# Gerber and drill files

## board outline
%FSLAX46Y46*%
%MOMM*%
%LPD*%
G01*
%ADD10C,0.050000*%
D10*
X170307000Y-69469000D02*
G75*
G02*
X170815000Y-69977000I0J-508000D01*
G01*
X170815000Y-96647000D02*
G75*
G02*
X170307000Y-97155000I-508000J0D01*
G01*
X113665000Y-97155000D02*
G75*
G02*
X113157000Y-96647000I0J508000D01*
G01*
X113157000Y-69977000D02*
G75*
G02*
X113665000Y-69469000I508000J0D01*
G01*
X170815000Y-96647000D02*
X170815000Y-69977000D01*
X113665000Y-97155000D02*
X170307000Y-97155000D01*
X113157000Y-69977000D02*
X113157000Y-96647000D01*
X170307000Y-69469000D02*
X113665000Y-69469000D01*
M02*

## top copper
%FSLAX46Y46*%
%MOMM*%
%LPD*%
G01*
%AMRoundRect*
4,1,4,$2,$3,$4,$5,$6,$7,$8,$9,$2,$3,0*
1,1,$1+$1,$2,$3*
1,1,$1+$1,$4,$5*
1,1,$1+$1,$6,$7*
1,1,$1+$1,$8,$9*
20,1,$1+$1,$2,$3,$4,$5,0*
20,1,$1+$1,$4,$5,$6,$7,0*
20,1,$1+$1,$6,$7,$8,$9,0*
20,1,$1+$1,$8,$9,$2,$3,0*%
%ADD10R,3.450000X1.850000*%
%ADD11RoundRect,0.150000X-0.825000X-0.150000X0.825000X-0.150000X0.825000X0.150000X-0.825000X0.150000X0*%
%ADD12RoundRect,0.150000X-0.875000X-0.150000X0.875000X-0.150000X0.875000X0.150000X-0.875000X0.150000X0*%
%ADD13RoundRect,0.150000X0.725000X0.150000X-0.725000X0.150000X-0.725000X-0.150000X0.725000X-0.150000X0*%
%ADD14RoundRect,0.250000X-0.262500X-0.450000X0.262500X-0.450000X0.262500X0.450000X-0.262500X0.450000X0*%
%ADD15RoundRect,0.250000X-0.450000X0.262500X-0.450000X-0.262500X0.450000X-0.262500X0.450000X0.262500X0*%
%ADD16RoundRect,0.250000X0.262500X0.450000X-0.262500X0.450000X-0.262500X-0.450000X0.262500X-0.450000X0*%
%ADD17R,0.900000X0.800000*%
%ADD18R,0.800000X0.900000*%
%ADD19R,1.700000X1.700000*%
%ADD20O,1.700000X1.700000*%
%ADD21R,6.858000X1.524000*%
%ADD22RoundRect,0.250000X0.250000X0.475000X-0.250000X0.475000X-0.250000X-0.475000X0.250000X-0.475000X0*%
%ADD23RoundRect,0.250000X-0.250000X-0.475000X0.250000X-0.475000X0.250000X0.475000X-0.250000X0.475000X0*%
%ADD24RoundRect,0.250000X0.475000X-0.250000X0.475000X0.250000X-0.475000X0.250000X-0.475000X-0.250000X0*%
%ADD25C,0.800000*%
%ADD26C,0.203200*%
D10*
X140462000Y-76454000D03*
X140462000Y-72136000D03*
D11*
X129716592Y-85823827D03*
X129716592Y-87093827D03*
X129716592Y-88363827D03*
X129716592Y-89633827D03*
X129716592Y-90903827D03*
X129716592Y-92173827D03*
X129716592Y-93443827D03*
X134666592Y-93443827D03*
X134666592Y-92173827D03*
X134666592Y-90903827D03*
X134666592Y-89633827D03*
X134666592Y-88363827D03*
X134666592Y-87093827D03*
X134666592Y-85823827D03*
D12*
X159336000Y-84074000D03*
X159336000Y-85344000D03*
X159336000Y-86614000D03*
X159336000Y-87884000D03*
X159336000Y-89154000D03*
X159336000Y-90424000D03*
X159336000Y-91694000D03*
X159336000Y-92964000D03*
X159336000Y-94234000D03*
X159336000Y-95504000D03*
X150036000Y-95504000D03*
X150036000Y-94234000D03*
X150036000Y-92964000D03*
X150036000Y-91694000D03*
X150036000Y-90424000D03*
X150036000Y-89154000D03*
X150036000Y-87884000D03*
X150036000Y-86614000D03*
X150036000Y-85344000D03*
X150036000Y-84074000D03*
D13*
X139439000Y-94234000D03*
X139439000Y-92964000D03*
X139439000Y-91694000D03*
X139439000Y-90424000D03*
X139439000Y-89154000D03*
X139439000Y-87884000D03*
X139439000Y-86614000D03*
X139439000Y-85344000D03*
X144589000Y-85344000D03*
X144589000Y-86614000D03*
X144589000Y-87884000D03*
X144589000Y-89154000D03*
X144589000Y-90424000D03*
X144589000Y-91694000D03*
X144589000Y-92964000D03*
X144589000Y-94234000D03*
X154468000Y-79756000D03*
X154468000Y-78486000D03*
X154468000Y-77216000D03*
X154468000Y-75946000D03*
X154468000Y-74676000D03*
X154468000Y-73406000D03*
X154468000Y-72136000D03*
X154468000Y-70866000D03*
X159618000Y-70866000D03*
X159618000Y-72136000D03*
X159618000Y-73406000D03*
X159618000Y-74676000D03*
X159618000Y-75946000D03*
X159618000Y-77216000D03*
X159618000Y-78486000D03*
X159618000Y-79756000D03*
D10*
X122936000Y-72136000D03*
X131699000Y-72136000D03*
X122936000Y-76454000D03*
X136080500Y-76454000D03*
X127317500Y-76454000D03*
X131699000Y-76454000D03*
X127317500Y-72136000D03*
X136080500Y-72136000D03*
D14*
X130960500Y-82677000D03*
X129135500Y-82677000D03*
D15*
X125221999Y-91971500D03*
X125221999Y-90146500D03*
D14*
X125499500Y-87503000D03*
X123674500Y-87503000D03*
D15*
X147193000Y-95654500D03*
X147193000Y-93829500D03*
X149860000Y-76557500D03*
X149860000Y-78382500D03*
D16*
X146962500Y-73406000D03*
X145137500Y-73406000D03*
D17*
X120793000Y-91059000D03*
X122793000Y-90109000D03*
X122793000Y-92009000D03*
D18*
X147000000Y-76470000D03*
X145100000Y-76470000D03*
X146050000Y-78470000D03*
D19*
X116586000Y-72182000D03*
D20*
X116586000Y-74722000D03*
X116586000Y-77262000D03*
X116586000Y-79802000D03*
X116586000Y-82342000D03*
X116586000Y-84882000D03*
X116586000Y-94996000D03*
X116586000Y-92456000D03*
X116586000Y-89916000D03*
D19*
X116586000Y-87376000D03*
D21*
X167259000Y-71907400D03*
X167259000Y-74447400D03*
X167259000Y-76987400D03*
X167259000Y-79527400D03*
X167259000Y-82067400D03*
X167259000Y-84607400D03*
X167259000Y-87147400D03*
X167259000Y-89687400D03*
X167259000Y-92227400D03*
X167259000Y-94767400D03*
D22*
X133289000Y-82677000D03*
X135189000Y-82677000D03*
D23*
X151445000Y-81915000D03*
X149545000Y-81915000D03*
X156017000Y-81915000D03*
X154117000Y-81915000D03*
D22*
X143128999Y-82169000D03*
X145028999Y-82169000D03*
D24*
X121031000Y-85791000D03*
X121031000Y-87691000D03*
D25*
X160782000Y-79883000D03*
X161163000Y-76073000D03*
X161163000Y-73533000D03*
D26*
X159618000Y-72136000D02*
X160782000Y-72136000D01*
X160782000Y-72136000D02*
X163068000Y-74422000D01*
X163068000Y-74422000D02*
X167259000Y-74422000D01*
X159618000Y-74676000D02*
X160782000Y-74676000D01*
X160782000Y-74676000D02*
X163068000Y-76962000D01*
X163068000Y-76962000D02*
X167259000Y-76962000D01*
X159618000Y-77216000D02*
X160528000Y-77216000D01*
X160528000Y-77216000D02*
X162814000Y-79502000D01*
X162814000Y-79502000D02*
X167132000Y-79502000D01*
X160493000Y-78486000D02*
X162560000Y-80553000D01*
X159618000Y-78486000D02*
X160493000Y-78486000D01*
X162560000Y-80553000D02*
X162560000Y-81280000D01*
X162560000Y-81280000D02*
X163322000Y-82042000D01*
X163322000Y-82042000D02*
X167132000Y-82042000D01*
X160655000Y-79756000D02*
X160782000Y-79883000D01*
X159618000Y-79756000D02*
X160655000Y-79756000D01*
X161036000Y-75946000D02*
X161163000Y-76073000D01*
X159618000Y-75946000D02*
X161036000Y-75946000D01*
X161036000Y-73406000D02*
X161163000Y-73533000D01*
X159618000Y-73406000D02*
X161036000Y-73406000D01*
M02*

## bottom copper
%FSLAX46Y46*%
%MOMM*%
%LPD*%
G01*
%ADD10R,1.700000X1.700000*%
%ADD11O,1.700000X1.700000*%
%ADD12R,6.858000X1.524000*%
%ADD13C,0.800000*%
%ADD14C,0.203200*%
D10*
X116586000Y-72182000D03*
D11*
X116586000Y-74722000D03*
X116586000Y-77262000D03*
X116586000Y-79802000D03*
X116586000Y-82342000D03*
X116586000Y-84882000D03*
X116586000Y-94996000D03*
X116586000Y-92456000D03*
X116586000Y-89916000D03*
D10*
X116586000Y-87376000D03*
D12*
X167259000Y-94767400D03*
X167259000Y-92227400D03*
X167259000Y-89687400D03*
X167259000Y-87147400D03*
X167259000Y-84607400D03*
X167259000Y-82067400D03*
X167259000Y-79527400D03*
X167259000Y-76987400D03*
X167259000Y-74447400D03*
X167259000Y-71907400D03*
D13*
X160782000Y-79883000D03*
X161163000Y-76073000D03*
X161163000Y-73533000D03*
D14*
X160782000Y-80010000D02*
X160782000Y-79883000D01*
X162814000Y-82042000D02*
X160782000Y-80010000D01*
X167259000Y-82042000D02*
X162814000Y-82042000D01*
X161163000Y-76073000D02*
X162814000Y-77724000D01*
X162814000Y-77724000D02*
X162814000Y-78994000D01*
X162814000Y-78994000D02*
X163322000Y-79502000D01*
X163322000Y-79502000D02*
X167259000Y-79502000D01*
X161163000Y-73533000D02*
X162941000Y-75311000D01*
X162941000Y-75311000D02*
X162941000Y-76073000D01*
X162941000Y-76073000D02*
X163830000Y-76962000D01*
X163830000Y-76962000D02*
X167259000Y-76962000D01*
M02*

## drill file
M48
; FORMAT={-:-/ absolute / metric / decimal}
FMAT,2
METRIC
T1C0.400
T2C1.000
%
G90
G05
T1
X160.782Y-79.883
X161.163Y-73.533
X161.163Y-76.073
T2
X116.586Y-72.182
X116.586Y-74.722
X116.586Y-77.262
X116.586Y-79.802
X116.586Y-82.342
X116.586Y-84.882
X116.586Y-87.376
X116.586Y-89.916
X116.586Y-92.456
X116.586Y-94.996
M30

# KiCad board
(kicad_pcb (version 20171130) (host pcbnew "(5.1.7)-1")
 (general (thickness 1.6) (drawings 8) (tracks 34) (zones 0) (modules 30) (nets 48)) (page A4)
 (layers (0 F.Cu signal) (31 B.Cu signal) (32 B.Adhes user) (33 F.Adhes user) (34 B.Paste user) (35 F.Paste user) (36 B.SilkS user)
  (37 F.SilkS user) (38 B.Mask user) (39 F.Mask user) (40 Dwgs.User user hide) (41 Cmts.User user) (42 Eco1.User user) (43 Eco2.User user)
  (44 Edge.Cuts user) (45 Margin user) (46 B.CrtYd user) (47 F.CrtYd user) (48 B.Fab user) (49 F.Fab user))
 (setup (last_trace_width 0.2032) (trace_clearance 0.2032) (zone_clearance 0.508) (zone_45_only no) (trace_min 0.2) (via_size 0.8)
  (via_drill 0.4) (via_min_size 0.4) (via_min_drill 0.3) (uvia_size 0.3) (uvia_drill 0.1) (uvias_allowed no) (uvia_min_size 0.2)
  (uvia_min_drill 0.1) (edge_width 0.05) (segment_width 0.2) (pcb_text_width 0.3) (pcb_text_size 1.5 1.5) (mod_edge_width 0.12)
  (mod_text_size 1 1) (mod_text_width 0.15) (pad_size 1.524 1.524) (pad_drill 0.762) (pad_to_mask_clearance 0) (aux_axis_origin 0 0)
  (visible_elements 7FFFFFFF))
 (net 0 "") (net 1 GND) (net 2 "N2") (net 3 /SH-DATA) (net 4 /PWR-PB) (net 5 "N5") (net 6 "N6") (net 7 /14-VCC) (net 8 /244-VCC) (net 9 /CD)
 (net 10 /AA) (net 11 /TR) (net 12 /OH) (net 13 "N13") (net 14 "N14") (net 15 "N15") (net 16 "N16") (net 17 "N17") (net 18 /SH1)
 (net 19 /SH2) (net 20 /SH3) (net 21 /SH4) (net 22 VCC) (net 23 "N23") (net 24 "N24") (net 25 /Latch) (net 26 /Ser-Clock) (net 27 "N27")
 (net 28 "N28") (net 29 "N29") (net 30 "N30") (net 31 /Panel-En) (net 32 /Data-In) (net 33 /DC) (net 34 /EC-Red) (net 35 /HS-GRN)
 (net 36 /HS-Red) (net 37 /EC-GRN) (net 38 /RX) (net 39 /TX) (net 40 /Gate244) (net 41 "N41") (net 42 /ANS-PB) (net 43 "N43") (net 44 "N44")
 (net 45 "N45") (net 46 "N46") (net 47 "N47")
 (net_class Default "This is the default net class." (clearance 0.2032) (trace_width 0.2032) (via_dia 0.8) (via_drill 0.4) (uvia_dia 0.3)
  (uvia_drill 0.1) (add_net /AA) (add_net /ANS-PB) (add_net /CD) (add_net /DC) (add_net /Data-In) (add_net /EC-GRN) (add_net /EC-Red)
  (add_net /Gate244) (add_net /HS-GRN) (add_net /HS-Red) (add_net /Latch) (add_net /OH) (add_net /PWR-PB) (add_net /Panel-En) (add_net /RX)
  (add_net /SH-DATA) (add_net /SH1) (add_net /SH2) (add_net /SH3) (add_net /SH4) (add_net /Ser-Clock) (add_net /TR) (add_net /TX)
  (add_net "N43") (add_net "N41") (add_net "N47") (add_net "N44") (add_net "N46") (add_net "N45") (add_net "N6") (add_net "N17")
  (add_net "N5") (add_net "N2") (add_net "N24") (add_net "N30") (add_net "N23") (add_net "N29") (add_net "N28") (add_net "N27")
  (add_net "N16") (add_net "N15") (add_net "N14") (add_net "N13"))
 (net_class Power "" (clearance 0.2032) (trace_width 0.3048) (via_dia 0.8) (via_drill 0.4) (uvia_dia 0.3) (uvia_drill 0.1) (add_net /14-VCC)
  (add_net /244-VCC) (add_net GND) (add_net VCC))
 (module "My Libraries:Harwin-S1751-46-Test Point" (layer F.Cu) (at 140.462 76.454)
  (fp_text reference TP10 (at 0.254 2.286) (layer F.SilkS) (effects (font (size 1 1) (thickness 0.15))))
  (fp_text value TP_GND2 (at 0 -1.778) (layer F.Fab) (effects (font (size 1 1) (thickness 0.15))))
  (pad 1 smd rect (at 0 0) (size 3.45 1.85) (layers F.Cu F.Paste F.Mask) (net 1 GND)))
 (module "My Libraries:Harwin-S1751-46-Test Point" (layer F.Cu) (at 140.462 72.136)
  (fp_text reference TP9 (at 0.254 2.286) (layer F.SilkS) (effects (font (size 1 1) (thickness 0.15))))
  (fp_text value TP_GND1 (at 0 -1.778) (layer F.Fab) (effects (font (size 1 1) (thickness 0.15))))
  (pad 1 smd rect (at 0 0) (size 3.45 1.85) (layers F.Cu F.Paste F.Mask) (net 1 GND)))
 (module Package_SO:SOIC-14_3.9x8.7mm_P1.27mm (layer F.Cu) (at 132.191592 89.633827)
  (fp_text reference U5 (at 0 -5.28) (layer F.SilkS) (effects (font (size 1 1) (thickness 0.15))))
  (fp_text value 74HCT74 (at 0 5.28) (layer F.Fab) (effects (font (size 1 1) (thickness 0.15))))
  (pad 1 smd roundrect (at -2.475 -3.81) (size 1.95 0.6) (layers F.Cu F.Paste F.Mask) (roundrect_rratio 0.25) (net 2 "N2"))
  (pad 2 smd roundrect (at -2.475 -2.54) (size 1.95 0.6) (layers F.Cu F.Paste F.Mask) (roundrect_rratio 0.25) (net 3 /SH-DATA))
  (pad 3 smd roundrect (at -2.475 -1.27) (size 1.95 0.6) (layers F.Cu F.Paste F.Mask) (roundrect_rratio 0.25) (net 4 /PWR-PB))
  (pad 4 smd roundrect (at -2.475 0) (size 1.95 0.6) (layers F.Cu F.Paste F.Mask) (roundrect_rratio 0.25) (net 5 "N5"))
  (pad 5 smd roundrect (at -2.475 1.27) (size 1.95 0.6) (layers F.Cu F.Paste F.Mask) (roundrect_rratio 0.25) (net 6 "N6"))
  (pad 6 smd roundrect (at -2.475 2.54) (size 1.95 0.6) (layers F.Cu F.Paste F.Mask) (roundrect_rratio 0.25) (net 3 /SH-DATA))
  (pad 7 smd roundrect (at -2.475 3.81) (size 1.95 0.6) (layers F.Cu F.Paste F.Mask) (roundrect_rratio 0.25) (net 1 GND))
  (pad 8 smd roundrect (at 2.475 3.81) (size 1.95 0.6) (layers F.Cu F.Paste F.Mask) (roundrect_rratio 0.25))
  (pad 9 smd roundrect (at 2.475 2.54) (size 1.95 0.6) (layers F.Cu F.Paste F.Mask) (roundrect_rratio 0.25))
  (pad 10 smd roundrect (at 2.475 1.27) (size 1.95 0.6) (layers F.Cu F.Paste F.Mask) (roundrect_rratio 0.25))
  (pad 11 smd roundrect (at 2.475 0) (size 1.95 0.6) (layers F.Cu F.Paste F.Mask) (roundrect_rratio 0.25))
  (pad 12 smd roundrect (at 2.475 -1.27) (size 1.95 0.6) (layers F.Cu F.Paste F.Mask) (roundrect_rratio 0.25))
  (pad 13 smd roundrect (at 2.475 -2.54) (size 1.95 0.6) (layers F.Cu F.Paste F.Mask) (roundrect_rratio 0.25))
  (pad 14 smd roundrect (at 2.475 -3.81) (size 1.95 0.6) (layers F.Cu F.Paste F.Mask) (roundrect_rratio 0.25) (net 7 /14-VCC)))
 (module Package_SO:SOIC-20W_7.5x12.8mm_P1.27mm (layer F.Cu) (at 154.686 89.789)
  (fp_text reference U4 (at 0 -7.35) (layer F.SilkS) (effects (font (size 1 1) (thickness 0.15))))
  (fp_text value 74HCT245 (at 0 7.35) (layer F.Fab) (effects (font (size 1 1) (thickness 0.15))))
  (pad 20 smd roundrect (at 4.65 -5.715) (size 2.05 0.6) (layers F.Cu F.Paste F.Mask) (roundrect_rratio 0.25) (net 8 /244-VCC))
  (pad 19 smd roundrect (at 4.65 -4.445) (size 2.05 0.6) (layers F.Cu F.Paste F.Mask) (roundrect_rratio 0.25) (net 1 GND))
  (pad 18 smd roundrect (at 4.65 -3.175) (size 2.05 0.6) (layers F.Cu F.Paste F.Mask) (roundrect_rratio 0.25) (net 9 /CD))
  (pad 17 smd roundrect (at 4.65 -1.905) (size 2.05 0.6) (layers F.Cu F.Paste F.Mask) (roundrect_rratio 0.25) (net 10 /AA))
  (pad 16 smd roundrect (at 4.65 -0.635) (size 2.05 0.6) (layers F.Cu F.Paste F.Mask) (roundrect_rratio 0.25) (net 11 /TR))
  (pad 15 smd roundrect (at 4.65 0.635) (size 2.05 0.6) (layers F.Cu F.Paste F.Mask) (roundrect_rratio 0.25) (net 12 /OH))
  (pad 14 smd roundrect (at 4.65 1.905) (size 2.05 0.6) (layers F.Cu F.Paste F.Mask) (roundrect_rratio 0.25) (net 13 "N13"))
  (pad 13 smd roundrect (at 4.65 3.175) (size 2.05 0.6) (layers F.Cu F.Paste F.Mask) (roundrect_rratio 0.25) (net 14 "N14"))
  (pad 12 smd roundrect (at 4.65 4.445) (size 2.05 0.6) (layers F.Cu F.Paste F.Mask) (roundrect_rratio 0.25) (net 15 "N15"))
  (pad 11 smd roundrect (at 4.65 5.715) (size 2.05 0.6) (layers F.Cu F.Paste F.Mask) (roundrect_rratio 0.25) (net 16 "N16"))
  (pad 10 smd roundrect (at -4.65 5.715) (size 2.05 0.6) (layers F.Cu F.Paste F.Mask) (roundrect_rratio 0.25) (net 1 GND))
  (pad 9 smd roundrect (at -4.65 4.445) (size 2.05 0.6) (layers F.Cu F.Paste F.Mask) (roundrect_rratio 0.25) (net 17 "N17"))
  (pad 8 smd roundrect (at -4.65 3.175) (size 2.05 0.6) (layers F.Cu F.Paste F.Mask) (roundrect_rratio 0.25) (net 17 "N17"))
  (pad 7 smd roundrect (at -4.65 1.905) (size 2.05 0.6) (layers F.Cu F.Paste F.Mask) (roundrect_rratio 0.25) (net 17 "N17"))
  (pad 6 smd roundrect (at -4.65 0.635) (size 2.05 0.6) (layers F.Cu F.Paste F.Mask) (roundrect_rratio 0.25) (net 17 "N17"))
  (pad 5 smd roundrect (at -4.65 -0.635) (size 2.05 0.6) (layers F.Cu F.Paste F.Mask) (roundrect_rratio 0.25) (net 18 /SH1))
  (pad 4 smd roundrect (at -4.65 -1.905) (size 2.05 0.6) (layers F.Cu F.Paste F.Mask) (roundrect_rratio 0.25) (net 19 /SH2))
  (pad 3 smd roundrect (at -4.65 -3.175) (size 2.05 0.6) (layers F.Cu F.Paste F.Mask) (roundrect_rratio 0.25) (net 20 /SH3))
  (pad 2 smd roundrect (at -4.65 -4.445) (size 2.05 0.6) (layers F.Cu F.Paste F.Mask) (roundrect_rratio 0.25) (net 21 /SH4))
  (pad 1 smd roundrect (at -4.65 -5.715) (size 2.05 0.6) (layers F.Cu F.Paste F.Mask) (roundrect_rratio 0.25) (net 8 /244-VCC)))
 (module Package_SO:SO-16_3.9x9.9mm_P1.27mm (layer F.Cu) (at 142.014 89.789 180)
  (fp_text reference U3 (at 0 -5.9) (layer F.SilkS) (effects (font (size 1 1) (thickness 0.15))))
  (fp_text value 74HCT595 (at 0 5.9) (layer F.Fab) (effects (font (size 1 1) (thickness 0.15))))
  (pad 16 smd roundrect (at 2.575 -4.445 180) (size 1.75 0.6) (layers F.Cu F.Paste F.Mask) (roundrect_rratio 0.25) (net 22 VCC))
  (pad 15 smd roundrect (at 2.575 -3.175 180) (size 1.75 0.6) (layers F.Cu F.Paste F.Mask) (roundrect_rratio 0.25) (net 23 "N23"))
  (pad 14 smd roundrect (at 2.575 -1.905 180) (size 1.75 0.6) (layers F.Cu F.Paste F.Mask) (roundrect_rratio 0.25) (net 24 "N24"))
  (pad 13 smd roundrect (at 2.575 -0.635 180) (size 1.75 0.6) (layers F.Cu F.Paste F.Mask) (roundrect_rratio 0.25) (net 1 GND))
  (pad 12 smd roundrect (at 2.575 0.635 180) (size 1.75 0.6) (layers F.Cu F.Paste F.Mask) (roundrect_rratio 0.25) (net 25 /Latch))
  (pad 11 smd roundrect (at 2.575 1.905 180) (size 1.75 0.6) (layers F.Cu F.Paste F.Mask) (roundrect_rratio 0.25) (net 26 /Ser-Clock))
  (pad 10 smd roundrect (at 2.575 3.175 180) (size 1.75 0.6) (layers F.Cu F.Paste F.Mask) (roundrect_rratio 0.25) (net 22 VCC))
  (pad 9 smd roundrect (at 2.575 4.445 180) (size 1.75 0.6) (layers F.Cu F.Paste F.Mask) (roundrect_rratio 0.25) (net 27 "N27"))
  (pad 8 smd roundrect (at -2.575 4.445 180) (size 1.75 0.6) (layers F.Cu F.Paste F.Mask) (roundrect_rratio 0.25) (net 1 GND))
  (pad 7 smd roundrect (at -2.575 3.175 180) (size 1.75 0.6) (layers F.Cu F.Paste F.Mask) (roundrect_rratio 0.25) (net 21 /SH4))
  (pad 6 smd roundrect (at -2.575 1.905 180) (size 1.75 0.6) (layers F.Cu F.Paste F.Mask) (roundrect_rratio 0.25) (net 20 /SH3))
  (pad 5 smd roundrect (at -2.575 0.635 180) (size 1.75 0.6) (layers F.Cu F.Paste F.Mask) (roundrect_rratio 0.25) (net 19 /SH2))
  (pad 4 smd roundrect (at -2.575 -0.635 180) (size 1.75 0.6) (layers F.Cu F.Paste F.Mask) (roundrect_rratio 0.25) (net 18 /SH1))
  (pad 3 smd roundrect (at -2.575 -1.905 180) (size 1.75 0.6) (layers F.Cu F.Paste F.Mask) (roundrect_rratio 0.25) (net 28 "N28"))
  (pad 2 smd roundrect (at -2.575 -3.175 180) (size 1.75 0.6) (layers F.Cu F.Paste F.Mask) (roundrect_rratio 0.25) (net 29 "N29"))
  (pad 1 smd roundrect (at -2.575 -4.445 180) (size 1.75 0.6) (layers F.Cu F.Paste F.Mask) (roundrect_rratio 0.25) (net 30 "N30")))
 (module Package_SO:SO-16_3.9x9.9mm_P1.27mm (layer F.Cu) (at 157.043 75.311 180)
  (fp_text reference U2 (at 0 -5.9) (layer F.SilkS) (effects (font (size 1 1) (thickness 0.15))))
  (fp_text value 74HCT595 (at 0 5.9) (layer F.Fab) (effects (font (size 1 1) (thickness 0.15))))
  (pad 16 smd roundrect (at 2.575 -4.445 180) (size 1.75 0.6) (layers F.Cu F.Paste F.Mask) (roundrect_rratio 0.25) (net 22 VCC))
  (pad 15 smd roundrect (at 2.575 -3.175 180) (size 1.75 0.6) (layers F.Cu F.Paste F.Mask) (roundrect_rratio 0.25) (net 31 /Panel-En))
  (pad 14 smd roundrect (at 2.575 -1.905 180) (size 1.75 0.6) (layers F.Cu F.Paste F.Mask) (roundrect_rratio 0.25) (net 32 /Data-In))
  (pad 13 smd roundrect (at 2.575 -0.635 180) (size 1.75 0.6) (layers F.Cu F.Paste F.Mask) (roundrect_rratio 0.25) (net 1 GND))
  (pad 12 smd roundrect (at 2.575 0.635 180) (size 1.75 0.6) (layers F.Cu F.Paste F.Mask) (roundrect_rratio 0.25) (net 25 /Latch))
  (pad 11 smd roundrect (at 2.575 1.905 180) (size 1.75 0.6) (layers F.Cu F.Paste F.Mask) (roundrect_rratio 0.25) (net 26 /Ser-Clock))
  (pad 10 smd roundrect (at 2.575 3.175 180) (size 1.75 0.6) (layers F.Cu F.Paste F.Mask) (roundrect_rratio 0.25) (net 22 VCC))
  (pad 9 smd roundrect (at 2.575 4.445 180) (size 1.75 0.6) (layers F.Cu F.Paste F.Mask) (roundrect_rratio 0.25) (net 24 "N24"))
  (pad 8 smd roundrect (at -2.575 4.445 180) (size 1.75 0.6) (layers F.Cu F.Paste F.Mask) (roundrect_rratio 0.25) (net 1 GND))
  (pad 7 smd roundrect (at -2.575 3.175 180) (size 1.75 0.6) (layers F.Cu F.Paste F.Mask) (roundrect_rratio 0.25) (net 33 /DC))
  (pad 6 smd roundrect (at -2.575 1.905 180) (size 1.75 0.6) (layers F.Cu F.Paste F.Mask) (roundrect_rratio 0.25) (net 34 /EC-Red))
  (pad 5 smd roundrect (at -2.575 0.635 180) (size 1.75 0.6) (layers F.Cu F.Paste F.Mask) (roundrect_rratio 0.25) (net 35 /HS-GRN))
  (pad 4 smd roundrect (at -2.575 -0.635 180) (size 1.75 0.6) (layers F.Cu F.Paste F.Mask) (roundrect_rratio 0.25) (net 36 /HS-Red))
  (pad 3 smd roundrect (at -2.575 -1.905 180) (size 1.75 0.6) (layers F.Cu F.Paste F.Mask) (roundrect_rratio 0.25) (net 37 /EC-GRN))
  (pad 2 smd roundrect (at -2.575 -3.175 180) (size 1.75 0.6) (layers F.Cu F.Paste F.Mask) (roundrect_rratio 0.25) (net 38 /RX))
  (pad 1 smd roundrect (at -2.575 -4.445 180) (size 1.75 0.6) (layers F.Cu F.Paste F.Mask) (roundrect_rratio 0.25) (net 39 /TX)))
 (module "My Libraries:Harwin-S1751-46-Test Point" (layer F.Cu) (at 122.936 72.136)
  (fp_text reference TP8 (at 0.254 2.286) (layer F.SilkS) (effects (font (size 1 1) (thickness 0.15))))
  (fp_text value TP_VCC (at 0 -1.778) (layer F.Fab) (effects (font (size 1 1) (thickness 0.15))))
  (pad 1 smd rect (at 0 0) (size 3.45 1.85) (layers F.Cu F.Paste F.Mask) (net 22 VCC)))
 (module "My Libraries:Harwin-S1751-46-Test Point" (layer F.Cu) (at 131.699 72.136)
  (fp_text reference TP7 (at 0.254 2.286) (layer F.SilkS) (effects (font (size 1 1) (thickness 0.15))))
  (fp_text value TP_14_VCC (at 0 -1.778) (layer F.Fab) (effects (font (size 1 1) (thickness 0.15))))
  (pad 1 smd rect (at 0 0) (size 3.45 1.85) (layers F.Cu F.Paste F.Mask) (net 7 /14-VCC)))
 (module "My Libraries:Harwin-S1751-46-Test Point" (layer F.Cu) (at 122.936 76.454)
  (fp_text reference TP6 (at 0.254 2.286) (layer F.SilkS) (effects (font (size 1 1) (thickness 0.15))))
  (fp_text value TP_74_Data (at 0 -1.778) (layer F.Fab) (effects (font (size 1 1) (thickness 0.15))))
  (pad 1 smd rect (at 0 0) (size 3.45 1.85) (layers F.Cu F.Paste F.Mask) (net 3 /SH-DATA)))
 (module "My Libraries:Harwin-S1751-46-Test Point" (layer F.Cu) (at 136.0805 76.454)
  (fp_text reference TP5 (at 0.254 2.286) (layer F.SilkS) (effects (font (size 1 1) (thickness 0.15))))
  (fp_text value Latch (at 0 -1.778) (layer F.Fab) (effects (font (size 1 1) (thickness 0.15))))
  (pad 1 smd rect (at 0 0) (size 3.45 1.85) (layers F.Cu F.Paste F.Mask) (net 25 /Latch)))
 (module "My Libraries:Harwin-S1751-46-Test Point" (layer F.Cu) (at 127.3175 76.454)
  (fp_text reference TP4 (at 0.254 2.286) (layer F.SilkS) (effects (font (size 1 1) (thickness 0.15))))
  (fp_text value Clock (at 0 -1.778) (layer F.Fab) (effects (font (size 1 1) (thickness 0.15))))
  (pad 1 smd rect (at 0 0) (size 3.45 1.85) (layers F.Cu F.Paste F.Mask) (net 26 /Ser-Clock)))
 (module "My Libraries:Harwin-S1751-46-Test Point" (layer F.Cu) (at 131.699 76.454)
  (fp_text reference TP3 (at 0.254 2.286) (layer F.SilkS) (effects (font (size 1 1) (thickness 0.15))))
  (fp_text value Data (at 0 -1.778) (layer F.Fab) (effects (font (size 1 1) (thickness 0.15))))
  (pad 1 smd rect (at 0 0) (size 3.45 1.85) (layers F.Cu F.Paste F.Mask) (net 32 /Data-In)))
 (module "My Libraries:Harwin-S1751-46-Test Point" (layer F.Cu) (at 127.3175 72.136)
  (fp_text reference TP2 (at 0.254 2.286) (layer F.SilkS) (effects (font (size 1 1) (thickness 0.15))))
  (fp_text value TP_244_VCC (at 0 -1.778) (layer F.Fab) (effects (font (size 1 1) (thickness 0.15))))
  (pad 1 smd rect (at 0 0) (size 3.45 1.85) (layers F.Cu F.Paste F.Mask) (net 8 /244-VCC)))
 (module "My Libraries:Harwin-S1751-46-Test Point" (layer F.Cu) (at 136.0805 72.136)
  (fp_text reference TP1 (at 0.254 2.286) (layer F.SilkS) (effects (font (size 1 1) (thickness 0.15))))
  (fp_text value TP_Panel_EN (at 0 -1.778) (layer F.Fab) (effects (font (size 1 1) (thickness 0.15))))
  (pad 1 smd rect (at 0 0) (size 3.45 1.85) (layers F.Cu F.Paste F.Mask) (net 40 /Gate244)))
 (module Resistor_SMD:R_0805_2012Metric (layer F.Cu) (at 130.048 82.677)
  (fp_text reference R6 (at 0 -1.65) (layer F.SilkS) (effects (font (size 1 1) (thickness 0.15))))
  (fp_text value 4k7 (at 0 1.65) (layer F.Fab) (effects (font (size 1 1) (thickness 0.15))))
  (pad 2 smd roundrect (at 0.9125 0) (size 1.025 1.4) (layers F.Cu F.Paste F.Mask) (roundrect_rratio 0.243902) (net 7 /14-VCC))
  (pad 1 smd roundrect (at -0.9125 0) (size 1.025 1.4) (layers F.Cu F.Paste F.Mask) (roundrect_rratio 0.243902) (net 2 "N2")))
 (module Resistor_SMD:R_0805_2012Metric (layer F.Cu) (at 125.221999 91.059 270)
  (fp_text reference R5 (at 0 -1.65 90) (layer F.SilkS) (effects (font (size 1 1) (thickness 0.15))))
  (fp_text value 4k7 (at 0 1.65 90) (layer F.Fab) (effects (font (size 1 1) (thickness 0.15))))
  (pad 2 smd roundrect (at 0.9125 0 270) (size 1.025 1.4) (layers F.Cu F.Paste F.Mask) (roundrect_rratio 0.243902) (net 6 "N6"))
  (pad 1 smd roundrect (at -0.9125 0 270) (size 1.025 1.4) (layers F.Cu F.Paste F.Mask) (roundrect_rratio 0.243902) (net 7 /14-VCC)))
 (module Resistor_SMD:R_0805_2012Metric (layer F.Cu) (at 124.587 87.503)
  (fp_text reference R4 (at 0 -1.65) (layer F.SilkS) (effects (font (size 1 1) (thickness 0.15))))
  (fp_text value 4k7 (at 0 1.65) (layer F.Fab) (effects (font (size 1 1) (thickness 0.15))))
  (pad 2 smd roundrect (at 0.9125 0) (size 1.025 1.4) (layers F.Cu F.Paste F.Mask) (roundrect_rratio 0.243902) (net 5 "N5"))
  (pad 1 smd roundrect (at -0.9125 0) (size 1.025 1.4) (layers F.Cu F.Paste F.Mask) (roundrect_rratio 0.243902) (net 7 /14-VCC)))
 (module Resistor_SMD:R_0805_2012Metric (layer F.Cu) (at 147.193 94.742 270)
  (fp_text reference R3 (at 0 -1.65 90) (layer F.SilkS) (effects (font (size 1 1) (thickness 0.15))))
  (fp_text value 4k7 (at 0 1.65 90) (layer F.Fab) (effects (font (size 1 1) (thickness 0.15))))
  (pad 2 smd roundrect (at 0.9125 0 270) (size 1.025 1.4) (layers F.Cu F.Paste F.Mask) (roundrect_rratio 0.243902) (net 1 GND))
  (pad 1 smd roundrect (at -0.9125 0 270) (size 1.025 1.4) (layers F.Cu F.Paste F.Mask) (roundrect_rratio 0.243902) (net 17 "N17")))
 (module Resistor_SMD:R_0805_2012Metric (layer F.Cu) (at 149.86 77.47 270)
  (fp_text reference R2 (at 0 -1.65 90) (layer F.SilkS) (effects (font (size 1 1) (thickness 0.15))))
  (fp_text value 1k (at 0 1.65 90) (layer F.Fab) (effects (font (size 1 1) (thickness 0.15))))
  (pad 1 smd roundrect (at -0.9125 0 270) (size 1.025 1.4) (layers F.Cu F.Paste F.Mask) (roundrect_rratio 0.243902) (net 40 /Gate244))
  (pad 2 smd roundrect (at 0.9125 0 270) (size 1.025 1.4) (layers F.Cu F.Paste F.Mask) (roundrect_rratio 0.243902) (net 31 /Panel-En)))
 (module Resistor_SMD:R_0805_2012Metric (layer F.Cu) (at 146.05 73.406 180)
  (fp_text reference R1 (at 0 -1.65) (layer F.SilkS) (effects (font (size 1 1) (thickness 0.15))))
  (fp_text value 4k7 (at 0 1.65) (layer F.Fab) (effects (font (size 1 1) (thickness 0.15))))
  (pad 1 smd roundrect (at -0.9125 0 180) (size 1.025 1.4) (layers F.Cu F.Paste F.Mask) (roundrect_rratio 0.243902) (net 40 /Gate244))
  (pad 2 smd roundrect (at 0.9125 0 180) (size 1.025 1.4) (layers F.Cu F.Paste F.Mask) (roundrect_rratio 0.243902) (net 22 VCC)))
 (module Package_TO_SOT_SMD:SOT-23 (layer F.Cu) (at 121.793 91.059 180)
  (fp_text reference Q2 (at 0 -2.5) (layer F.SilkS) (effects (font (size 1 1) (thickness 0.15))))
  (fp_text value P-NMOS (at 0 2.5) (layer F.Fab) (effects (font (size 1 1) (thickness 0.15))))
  (pad 3 smd rect (at 1 0 180) (size 0.9 0.8) (layers F.Cu F.Paste F.Mask) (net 22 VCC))
  (pad 2 smd rect (at -1 0.95 180) (size 0.9 0.8) (layers F.Cu F.Paste F.Mask) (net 7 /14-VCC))
  (pad 1 smd rect (at -1 -0.95 180) (size 0.9 0.8) (layers F.Cu F.Paste F.Mask) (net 6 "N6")))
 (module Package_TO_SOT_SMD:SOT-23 (layer F.Cu) (at 146.05 77.47 270)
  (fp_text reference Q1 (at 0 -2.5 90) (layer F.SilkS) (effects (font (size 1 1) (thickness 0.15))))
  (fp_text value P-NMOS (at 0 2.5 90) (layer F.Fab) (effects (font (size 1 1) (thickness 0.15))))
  (pad 1 smd rect (at -1 -0.95 270) (size 0.9 0.8) (layers F.Cu F.Paste F.Mask) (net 40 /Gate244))
  (pad 2 smd rect (at -1 0.95 270) (size 0.9 0.8) (layers F.Cu F.Paste F.Mask) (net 22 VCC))
  (pad 3 smd rect (at 1 0 270) (size 0.9 0.8) (layers F.Cu F.Paste F.Mask) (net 8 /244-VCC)))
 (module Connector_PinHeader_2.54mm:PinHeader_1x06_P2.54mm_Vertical (layer F.Cu) (at 116.586 72.182)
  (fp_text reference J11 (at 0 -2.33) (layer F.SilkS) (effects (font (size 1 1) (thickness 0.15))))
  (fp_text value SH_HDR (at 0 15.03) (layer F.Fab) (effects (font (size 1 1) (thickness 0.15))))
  (pad 1 thru_hole rect (at 0 0) (size 1.7 1.7) (drill 1) (layers *.Cu *.Mask) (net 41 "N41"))
  (pad 2 thru_hole oval (at 0 2.54) (size 1.7 1.7) (drill 1) (layers *.Cu *.Mask) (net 32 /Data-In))
  (pad 3 thru_hole oval (at 0 5.08) (size 1.7 1.7) (drill 1) (layers *.Cu *.Mask) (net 26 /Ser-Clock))
  (pad 4 thru_hole oval (at 0 7.62) (size 1.7 1.7) (drill 1) (layers *.Cu *.Mask) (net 25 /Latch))
  (pad 5 thru_hole oval (at 0 10.16) (size 1.7 1.7) (drill 1) (layers *.Cu *.Mask) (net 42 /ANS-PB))
  (pad 6 thru_hole oval (at 0 12.7) (size 1.7 1.7) (drill 1) (layers *.Cu *.Mask) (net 1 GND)))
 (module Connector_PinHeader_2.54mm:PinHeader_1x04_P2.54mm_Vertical (layer F.Cu) (at 116.586 87.376)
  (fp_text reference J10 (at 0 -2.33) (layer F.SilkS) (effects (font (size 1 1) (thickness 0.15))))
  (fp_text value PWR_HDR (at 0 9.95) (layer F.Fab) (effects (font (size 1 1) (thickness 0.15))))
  (pad 4 thru_hole oval (at 0 7.62) (size 1.7 1.7) (drill 1) (layers *.Cu *.Mask) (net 1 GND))
  (pad 3 thru_hole oval (at 0 5.08) (size 1.7 1.7) (drill 1) (layers *.Cu *.Mask) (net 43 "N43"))
  (pad 2 thru_hole oval (at 0 2.54) (size 1.7 1.7) (drill 1) (layers *.Cu *.Mask) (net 7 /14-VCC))
  (pad 1 thru_hole rect (at 0 0) (size 1.7 1.7) (drill 1) (layers *.Cu *.Mask) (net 22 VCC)))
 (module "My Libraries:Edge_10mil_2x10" (layer B.Cu) (at 167.259 83.3374 180)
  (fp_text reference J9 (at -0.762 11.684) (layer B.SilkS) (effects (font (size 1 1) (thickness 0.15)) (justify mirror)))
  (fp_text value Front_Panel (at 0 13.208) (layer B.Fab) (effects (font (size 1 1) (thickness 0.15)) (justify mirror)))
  (pad 20 connect rect (at 0 11.43 180) (size 6.858 1.524) (layers F.Cu B.Mask) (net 8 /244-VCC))
  (pad 19 connect rect (at 0 8.89 180) (size 6.858 1.524) (layers F.Cu B.Mask) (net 33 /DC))
  (pad 18 connect rect (at 0 6.35 180) (size 6.858 1.524) (layers F.Cu B.Mask) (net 35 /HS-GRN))
  (pad 17 connect rect (at 0 3.81 180) (size 6.858 1.524) (layers F.Cu B.Mask) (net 37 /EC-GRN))
  (pad 16 connect rect (at 0 1.27 180) (size 6.858 1.524) (layers F.Cu B.Mask) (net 38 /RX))
  (pad 15 connect rect (at 0 -1.27 180) (size 6.858 1.524) (layers F.Cu B.Mask) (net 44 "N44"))
  (pad 14 connect rect (at 0 -3.81 180) (size 6.858 1.524) (layers F.Cu B.Mask) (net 10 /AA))
  (pad 13 connect rect (at 0 -6.35 180) (size 6.858 1.524) (layers F.Cu B.Mask) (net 12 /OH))
  (pad 12 connect rect (at 0 -8.89 180) (size 6.858 1.524) (layers F.Cu B.Mask) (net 7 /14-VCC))
  (pad 11 connect rect (at 0 -11.43 180) (size 6.858 1.524) (layers F.Cu B.Mask) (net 1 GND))
  (pad 10 connect rect (at 0 -11.43 180) (size 6.858 1.524) (layers B.Cu B.Mask) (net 42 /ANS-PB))
  (pad 9 connect rect (at 0 -8.89 180) (size 6.858 1.524) (layers B.Cu B.Mask) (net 4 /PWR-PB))
  (pad 8 connect rect (at 0 -6.35 180) (size 6.858 1.524) (layers B.Cu B.Mask) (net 11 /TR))
  (pad 7 connect rect (at 0 -3.81 180) (size 6.858 1.524) (layers B.Cu B.Mask) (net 9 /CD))
  (pad 6 connect rect (at 0 -1.27 180) (size 6.858 1.524) (layers B.Cu B.Mask) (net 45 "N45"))
  (pad 5 connect rect (at 0 1.27 180) (size 6.858 1.524) (layers B.Cu B.Mask) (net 39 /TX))
  (pad 4 connect rect (at 0 3.81 180) (size 6.858 1.524) (layers B.Cu B.Mask) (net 36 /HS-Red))
  (pad 3 connect rect (at 0 6.35 180) (size 6.858 1.524) (layers B.Cu B.Mask) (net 34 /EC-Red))
  (pad 2 connect rect (at 0 8.89 180) (size 6.858 1.524) (layers B.Cu B.Mask) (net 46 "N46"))
  (pad 1 connect rect (at 0 11.43 180) (size 6.858 1.524) (layers B.Cu B.Mask) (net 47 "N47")))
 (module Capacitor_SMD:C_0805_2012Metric (layer F.Cu) (at 134.239 82.677 180)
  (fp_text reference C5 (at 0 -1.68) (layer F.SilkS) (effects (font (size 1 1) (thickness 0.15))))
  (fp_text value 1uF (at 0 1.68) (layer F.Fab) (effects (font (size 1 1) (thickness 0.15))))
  (pad 2 smd roundrect (at 0.95 0 180) (size 1 1.45) (layers F.Cu F.Paste F.Mask) (roundrect_rratio 0.25) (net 1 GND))
  (pad 1 smd roundrect (at -0.95 0 180) (size 1 1.45) (layers F.Cu F.Paste F.Mask) (roundrect_rratio 0.25) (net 7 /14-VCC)))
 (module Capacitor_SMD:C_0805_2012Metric (layer F.Cu) (at 150.495 81.915)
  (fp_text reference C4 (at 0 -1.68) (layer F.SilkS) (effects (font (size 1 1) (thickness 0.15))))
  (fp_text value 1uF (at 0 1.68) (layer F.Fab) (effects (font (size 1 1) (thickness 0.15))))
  (pad 2 smd roundrect (at 0.95 0) (size 1 1.45) (layers F.Cu F.Paste F.Mask) (roundrect_rratio 0.25) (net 1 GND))
  (pad 1 smd roundrect (at -0.95 0) (size 1 1.45) (layers F.Cu F.Paste F.Mask) (roundrect_rratio 0.25) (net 22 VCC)))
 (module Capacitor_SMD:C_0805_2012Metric (layer F.Cu) (at 155.067 81.915)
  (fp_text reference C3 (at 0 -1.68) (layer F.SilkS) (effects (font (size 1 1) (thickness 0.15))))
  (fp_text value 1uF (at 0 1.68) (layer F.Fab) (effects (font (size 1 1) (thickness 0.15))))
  (pad 2 smd roundrect (at 0.95 0) (size 1 1.45) (layers F.Cu F.Paste F.Mask) (roundrect_rratio 0.25) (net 1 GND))
  (pad 1 smd roundrect (at -0.95 0) (size 1 1.45) (layers F.Cu F.Paste F.Mask) (roundrect_rratio 0.25) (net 22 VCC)))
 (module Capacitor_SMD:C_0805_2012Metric (layer F.Cu) (at 144.078999 82.169 180)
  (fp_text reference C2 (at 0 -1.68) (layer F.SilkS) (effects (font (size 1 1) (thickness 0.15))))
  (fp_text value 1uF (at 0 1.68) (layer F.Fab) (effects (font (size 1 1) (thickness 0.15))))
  (pad 2 smd roundrect (at 0.95 0 180) (size 1 1.45) (layers F.Cu F.Paste F.Mask) (roundrect_rratio 0.25) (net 1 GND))
  (pad 1 smd roundrect (at -0.95 0 180) (size 1 1.45) (layers F.Cu F.Paste F.Mask) (roundrect_rratio 0.25) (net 22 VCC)))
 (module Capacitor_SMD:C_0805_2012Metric (layer F.Cu) (at 121.031 86.741 90)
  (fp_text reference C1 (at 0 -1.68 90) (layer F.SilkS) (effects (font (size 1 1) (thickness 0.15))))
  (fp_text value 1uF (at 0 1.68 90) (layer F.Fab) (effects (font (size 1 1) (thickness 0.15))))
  (pad 2 smd roundrect (at 0.95 0 90) (size 1 1.45) (layers F.Cu F.Paste F.Mask) (roundrect_rratio 0.25) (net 1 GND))
  (pad 1 smd roundrect (at -0.95 0 90) (size 1 1.45) (layers F.Cu F.Paste F.Mask) (roundrect_rratio 0.25) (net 22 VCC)))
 (gr_arc (start 170.307 69.977) (end 170.815 69.977) (angle -90) (layer Edge.Cuts) (width 0.05))
 (gr_arc (start 170.307 96.647) (end 170.307 97.155) (angle -90) (layer Edge.Cuts) (width 0.05))
 (gr_arc (start 113.665 96.647) (end 113.157 96.647) (angle -90) (layer Edge.Cuts) (width 0.05))
 (gr_arc (start 113.665 69.977) (end 113.665 69.469) (angle -90) (layer Edge.Cuts) (width 0.05))
 (gr_line (start 170.815 96.647) (end 170.815 69.977) (layer Edge.Cuts) (width 0.05))
 (gr_line (start 113.665 97.155) (end 170.307 97.155) (layer Edge.Cuts) (width 0.05))
 (gr_line (start 113.157 69.977) (end 113.157 96.647) (layer Edge.Cuts) (width 0.05))
 (gr_line (start 170.307 69.469) (end 113.665 69.469) (layer Edge.Cuts) (width 0.05))
 (segment (start 159.618 72.136) (end 160.782 72.136) (width 0.2032) (layer F.Cu) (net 33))
 (segment (start 160.782 72.136) (end 163.068 74.422) (width 0.2032) (layer F.Cu) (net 33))
 (segment (start 163.068 74.422) (end 167.259 74.422) (width 0.2032) (layer F.Cu) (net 33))
 (segment (start 159.618 74.676) (end 160.782 74.676) (width 0.2032) (layer F.Cu) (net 35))
 (segment (start 160.782 74.676) (end 163.068 76.962) (width 0.2032) (layer F.Cu) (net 35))
 (segment (start 163.068 76.962) (end 167.259 76.962) (width 0.2032) (layer F.Cu) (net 35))
 (segment (start 159.618 77.216) (end 160.528 77.216) (width 0.2032) (layer F.Cu) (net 37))
 (segment (start 160.528 77.216) (end 162.814 79.502) (width 0.2032) (layer F.Cu) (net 37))
 (segment (start 162.814 79.502) (end 167.132 79.502) (width 0.2032) (layer F.Cu) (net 37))
 (segment (start 160.493 78.486) (end 162.56 80.553) (width 0.2032) (layer F.Cu) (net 38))
 (segment (start 159.618 78.486) (end 160.493 78.486) (width 0.2032) (layer F.Cu) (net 38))
 (segment (start 162.56 80.553) (end 162.56 81.28) (width 0.2032) (layer F.Cu) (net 38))
 (segment (start 162.56 81.28) (end 163.322 82.042) (width 0.2032) (layer F.Cu) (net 38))
 (segment (start 163.322 82.042) (end 167.132 82.042) (width 0.2032) (layer F.Cu) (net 38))
 (segment (start 160.655 79.756) (end 160.782 79.883) (width 0.2032) (layer F.Cu) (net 39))
 (via (at 160.782 79.883) (size 0.8) (drill 0.4) (layers F.Cu B.Cu) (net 39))
 (segment (start 159.618 79.756) (end 160.655 79.756) (width 0.2032) (layer F.Cu) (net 39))
 (segment (start 160.782 80.01) (end 160.782 79.883) (width 0.2032) (layer B.Cu) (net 39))
 (segment (start 162.814 82.042) (end 160.782 80.01) (width 0.2032) (layer B.Cu) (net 39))
 (segment (start 167.259 82.042) (end 162.814 82.042) (width 0.2032) (layer B.Cu) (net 39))
 (via (at 161.163 76.073) (size 0.8) (drill 0.4) (layers F.Cu B.Cu) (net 36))
 (segment (start 161.036 75.946) (end 161.163 76.073) (width 0.2032) (layer F.Cu) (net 36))
 (segment (start 159.618 75.946) (end 161.036 75.946) (width 0.2032) (layer F.Cu) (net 36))
 (segment (start 161.163 76.073) (end 162.814 77.724) (width 0.2032) (layer B.Cu) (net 36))
 (segment (start 162.814 77.724) (end 162.814 78.994) (width 0.2032) (layer B.Cu) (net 36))
 (segment (start 162.814 78.994) (end 163.322 79.502) (width 0.2032) (layer B.Cu) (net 36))
 (segment (start 163.322 79.502) (end 167.259 79.502) (width 0.2032) (layer B.Cu) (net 36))
 (via (at 161.163 73.533) (size 0.8) (drill 0.4) (layers F.Cu B.Cu) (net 34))
 (segment (start 161.036 73.406) (end 161.163 73.533) (width 0.2032) (layer F.Cu) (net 34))
 (segment (start 159.618 73.406) (end 161.036 73.406) (width 0.2032) (layer F.Cu) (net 34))
 (segment (start 161.163 73.533) (end 162.941 75.311) (width 0.2032) (layer B.Cu) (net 34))
 (segment (start 162.941 75.311) (end 162.941 76.073) (width 0.2032) (layer B.Cu) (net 34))
 (segment (start 162.941 76.073) (end 163.83 76.962) (width 0.2032) (layer B.Cu) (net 34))
 (segment (start 163.83 76.962) (end 167.259 76.962) (width 0.2032) (layer B.Cu) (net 34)))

